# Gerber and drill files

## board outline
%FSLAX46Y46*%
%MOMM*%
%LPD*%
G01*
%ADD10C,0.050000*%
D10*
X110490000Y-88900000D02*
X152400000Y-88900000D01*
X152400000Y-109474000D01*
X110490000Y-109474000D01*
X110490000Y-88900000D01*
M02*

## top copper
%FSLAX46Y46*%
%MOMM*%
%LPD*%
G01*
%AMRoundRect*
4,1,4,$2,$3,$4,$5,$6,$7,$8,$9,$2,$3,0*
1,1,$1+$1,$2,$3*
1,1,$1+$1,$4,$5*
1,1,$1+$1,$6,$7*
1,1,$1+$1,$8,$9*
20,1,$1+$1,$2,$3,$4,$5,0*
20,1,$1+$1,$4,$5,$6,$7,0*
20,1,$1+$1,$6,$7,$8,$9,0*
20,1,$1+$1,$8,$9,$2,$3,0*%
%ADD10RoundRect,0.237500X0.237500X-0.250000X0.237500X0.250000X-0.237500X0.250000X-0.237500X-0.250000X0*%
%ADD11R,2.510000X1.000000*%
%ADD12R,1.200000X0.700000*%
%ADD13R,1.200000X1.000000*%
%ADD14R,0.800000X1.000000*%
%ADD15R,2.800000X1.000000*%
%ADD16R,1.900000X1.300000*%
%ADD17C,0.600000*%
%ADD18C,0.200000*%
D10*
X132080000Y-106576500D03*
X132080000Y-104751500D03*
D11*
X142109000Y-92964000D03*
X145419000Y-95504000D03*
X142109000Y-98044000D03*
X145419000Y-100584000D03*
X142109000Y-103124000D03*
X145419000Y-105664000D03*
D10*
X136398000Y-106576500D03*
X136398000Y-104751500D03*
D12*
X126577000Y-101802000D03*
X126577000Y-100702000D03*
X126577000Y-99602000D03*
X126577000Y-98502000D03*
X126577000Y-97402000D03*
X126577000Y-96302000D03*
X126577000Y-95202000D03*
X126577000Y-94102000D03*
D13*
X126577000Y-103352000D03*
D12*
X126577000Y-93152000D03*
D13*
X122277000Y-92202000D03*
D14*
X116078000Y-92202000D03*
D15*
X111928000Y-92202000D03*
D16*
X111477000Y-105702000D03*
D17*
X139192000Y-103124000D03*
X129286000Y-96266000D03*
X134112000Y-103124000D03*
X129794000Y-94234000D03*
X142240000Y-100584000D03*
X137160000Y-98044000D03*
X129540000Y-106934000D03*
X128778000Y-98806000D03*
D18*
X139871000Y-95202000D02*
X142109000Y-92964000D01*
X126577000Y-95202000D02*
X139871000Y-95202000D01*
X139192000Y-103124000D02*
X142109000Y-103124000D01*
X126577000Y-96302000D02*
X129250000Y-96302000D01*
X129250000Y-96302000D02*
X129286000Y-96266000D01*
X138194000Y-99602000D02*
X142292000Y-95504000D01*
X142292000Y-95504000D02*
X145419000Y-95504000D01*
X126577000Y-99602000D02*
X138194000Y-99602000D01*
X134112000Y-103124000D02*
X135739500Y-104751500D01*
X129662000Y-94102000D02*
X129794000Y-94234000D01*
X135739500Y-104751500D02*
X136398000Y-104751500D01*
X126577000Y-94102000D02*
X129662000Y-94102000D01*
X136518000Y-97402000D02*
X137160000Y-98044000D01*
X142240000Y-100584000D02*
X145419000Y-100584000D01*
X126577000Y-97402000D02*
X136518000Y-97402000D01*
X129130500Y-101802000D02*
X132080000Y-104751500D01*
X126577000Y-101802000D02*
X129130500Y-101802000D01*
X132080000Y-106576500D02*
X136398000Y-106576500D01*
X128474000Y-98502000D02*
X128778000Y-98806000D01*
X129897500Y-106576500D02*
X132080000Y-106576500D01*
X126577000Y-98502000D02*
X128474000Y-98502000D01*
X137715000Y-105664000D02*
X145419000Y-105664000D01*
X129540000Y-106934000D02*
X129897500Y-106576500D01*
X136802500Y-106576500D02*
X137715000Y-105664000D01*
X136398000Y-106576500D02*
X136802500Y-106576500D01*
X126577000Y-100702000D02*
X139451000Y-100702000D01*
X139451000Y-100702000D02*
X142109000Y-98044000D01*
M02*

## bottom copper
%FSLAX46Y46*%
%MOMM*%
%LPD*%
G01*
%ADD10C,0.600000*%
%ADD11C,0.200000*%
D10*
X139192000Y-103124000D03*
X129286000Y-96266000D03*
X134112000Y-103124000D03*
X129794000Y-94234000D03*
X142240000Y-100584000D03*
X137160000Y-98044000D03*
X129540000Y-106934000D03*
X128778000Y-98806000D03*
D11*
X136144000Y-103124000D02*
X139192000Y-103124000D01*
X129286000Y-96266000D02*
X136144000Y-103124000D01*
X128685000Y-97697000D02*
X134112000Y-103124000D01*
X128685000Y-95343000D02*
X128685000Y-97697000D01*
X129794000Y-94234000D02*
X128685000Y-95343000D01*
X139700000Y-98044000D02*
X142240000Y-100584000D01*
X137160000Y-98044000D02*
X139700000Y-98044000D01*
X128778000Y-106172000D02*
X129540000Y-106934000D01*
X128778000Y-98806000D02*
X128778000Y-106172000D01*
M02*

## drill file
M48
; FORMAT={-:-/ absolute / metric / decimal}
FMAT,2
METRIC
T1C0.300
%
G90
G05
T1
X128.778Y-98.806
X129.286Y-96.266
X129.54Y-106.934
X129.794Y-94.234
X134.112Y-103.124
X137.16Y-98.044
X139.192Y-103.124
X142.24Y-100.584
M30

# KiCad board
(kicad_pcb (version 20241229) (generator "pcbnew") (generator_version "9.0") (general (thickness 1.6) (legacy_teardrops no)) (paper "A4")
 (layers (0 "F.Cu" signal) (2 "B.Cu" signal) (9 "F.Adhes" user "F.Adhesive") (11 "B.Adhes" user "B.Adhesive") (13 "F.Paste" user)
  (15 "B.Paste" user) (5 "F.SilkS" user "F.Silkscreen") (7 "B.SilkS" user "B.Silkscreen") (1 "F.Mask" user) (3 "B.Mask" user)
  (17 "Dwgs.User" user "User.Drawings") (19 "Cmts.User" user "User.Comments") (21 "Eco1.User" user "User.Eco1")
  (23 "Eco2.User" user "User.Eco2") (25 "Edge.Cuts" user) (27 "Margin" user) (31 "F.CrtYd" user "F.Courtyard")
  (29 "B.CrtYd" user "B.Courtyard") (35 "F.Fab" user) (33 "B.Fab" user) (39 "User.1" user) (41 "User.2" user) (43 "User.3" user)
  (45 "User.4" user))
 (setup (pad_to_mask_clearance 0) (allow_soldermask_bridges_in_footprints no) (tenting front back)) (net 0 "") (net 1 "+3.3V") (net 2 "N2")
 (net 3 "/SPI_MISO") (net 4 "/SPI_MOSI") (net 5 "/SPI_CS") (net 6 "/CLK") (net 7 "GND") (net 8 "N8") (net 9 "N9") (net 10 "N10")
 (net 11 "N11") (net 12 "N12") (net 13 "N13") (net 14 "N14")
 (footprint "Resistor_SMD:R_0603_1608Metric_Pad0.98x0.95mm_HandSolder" (layer "F.Cu") (at 132.08 105.664 90)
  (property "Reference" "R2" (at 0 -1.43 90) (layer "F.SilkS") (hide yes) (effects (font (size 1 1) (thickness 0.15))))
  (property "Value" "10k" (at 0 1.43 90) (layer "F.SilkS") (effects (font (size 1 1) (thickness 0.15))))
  (pad "1" smd roundrect (at -0.9125 0 90) (size 0.975 0.95) (layers "F.Cu" "F.Mask" "F.Paste") (roundrect_rratio 0.25) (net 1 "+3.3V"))
  (pad "2" smd roundrect (at 0.9125 0 90) (size 0.975 0.95) (layers "F.Cu" "F.Mask" "F.Paste") (roundrect_rratio 0.25) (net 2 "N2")))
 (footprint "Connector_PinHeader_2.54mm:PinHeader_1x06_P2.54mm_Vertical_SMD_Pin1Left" (layer "F.Cu") (at 143.764 99.314)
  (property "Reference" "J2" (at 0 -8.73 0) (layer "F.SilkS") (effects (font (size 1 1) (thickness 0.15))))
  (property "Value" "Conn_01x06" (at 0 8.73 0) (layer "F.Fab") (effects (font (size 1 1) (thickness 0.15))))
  (pad "1" smd rect (at -1.655 -6.35) (size 2.51 1) (layers "F.Cu" "F.Mask" "F.Paste") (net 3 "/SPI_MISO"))
  (pad "2" smd rect (at 1.655 -3.81) (size 2.51 1) (layers "F.Cu" "F.Mask" "F.Paste") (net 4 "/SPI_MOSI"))
  (pad "3" smd rect (at -1.655 -1.27) (size 2.51 1) (layers "F.Cu" "F.Mask" "F.Paste") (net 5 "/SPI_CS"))
  (pad "4" smd rect (at 1.655 1.27) (size 2.51 1) (layers "F.Cu" "F.Mask" "F.Paste") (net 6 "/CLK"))
  (pad "5" smd rect (at -1.655 3.81) (size 2.51 1) (layers "F.Cu" "F.Mask" "F.Paste") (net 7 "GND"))
  (pad "6" smd rect (at 1.655 6.35) (size 2.51 1) (layers "F.Cu" "F.Mask" "F.Paste") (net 1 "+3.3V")))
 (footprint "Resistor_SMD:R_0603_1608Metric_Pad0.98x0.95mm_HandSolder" (layer "F.Cu") (at 136.398 105.664 90)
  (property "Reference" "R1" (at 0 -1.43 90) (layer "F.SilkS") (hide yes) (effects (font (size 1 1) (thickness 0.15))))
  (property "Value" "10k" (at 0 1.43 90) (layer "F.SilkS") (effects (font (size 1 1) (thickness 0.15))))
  (pad "1" smd roundrect (at -0.9125 0 90) (size 0.975 0.95) (layers "F.Cu" "F.Mask" "F.Paste") (roundrect_rratio 0.25) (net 1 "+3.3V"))
  (pad "2" smd roundrect (at 0.9125 0 90) (size 0.975 0.95) (layers "F.Cu" "F.Mask" "F.Paste") (roundrect_rratio 0.25) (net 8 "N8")))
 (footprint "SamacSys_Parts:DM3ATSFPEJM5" (layer "F.Cu") (at 119.165 99.027 -90)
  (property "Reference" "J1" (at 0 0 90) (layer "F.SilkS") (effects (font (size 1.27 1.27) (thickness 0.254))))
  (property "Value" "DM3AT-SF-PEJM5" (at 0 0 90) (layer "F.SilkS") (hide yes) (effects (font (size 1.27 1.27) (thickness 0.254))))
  (pad "1" smd rect (at 2.775 -7.412 270) (size 0.7 1.2) (layers "F.Cu" "F.Mask" "F.Paste") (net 2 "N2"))
  (pad "2" smd rect (at 1.675 -7.412 270) (size 0.7 1.2) (layers "F.Cu" "F.Mask" "F.Paste") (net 5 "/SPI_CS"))
  (pad "3" smd rect (at 0.575 -7.412 270) (size 0.7 1.2) (layers "F.Cu" "F.Mask" "F.Paste") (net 4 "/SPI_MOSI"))
  (pad "4" smd rect (at -0.525 -7.412 270) (size 0.7 1.2) (layers "F.Cu" "F.Mask" "F.Paste") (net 1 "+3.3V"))
  (pad "5" smd rect (at -1.625 -7.412 270) (size 0.7 1.2) (layers "F.Cu" "F.Mask" "F.Paste") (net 6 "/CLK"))
  (pad "6" smd rect (at -2.725 -7.412 270) (size 0.7 1.2) (layers "F.Cu" "F.Mask" "F.Paste") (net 7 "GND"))
  (pad "7" smd rect (at -3.825 -7.412 270) (size 0.7 1.2) (layers "F.Cu" "F.Mask" "F.Paste") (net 3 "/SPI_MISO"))
  (pad "8" smd rect (at -4.925 -7.412 270) (size 0.7 1.2) (layers "F.Cu" "F.Mask" "F.Paste") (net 8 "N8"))
  (pad "MP1" smd rect (at 4.325 -7.412 270) (size 1 1.2) (layers "F.Cu" "F.Mask" "F.Paste") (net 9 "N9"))
  (pad "MP2" smd rect (at -5.875 -7.412 270) (size 0.7 1.2) (layers "F.Cu" "F.Mask" "F.Paste") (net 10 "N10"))
  (pad "MP3" smd rect (at -6.825 -3.112 270) (size 1 1.2) (layers "F.Cu" "F.Mask" "F.Paste") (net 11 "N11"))
  (pad "MP4" smd rect (at -6.825 3.087) (size 0.8 1) (layers "F.Cu" "F.Mask" "F.Paste") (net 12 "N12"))
  (pad "MP5" smd rect (at -6.825 7.237 270) (size 1 2.8) (layers "F.Cu" "F.Mask" "F.Paste") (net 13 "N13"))
  (pad "MP6" smd rect (at 6.675 7.688 270) (size 1.3 1.9) (layers "F.Cu" "F.Mask" "F.Paste") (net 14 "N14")))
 (gr_rect (start 110.49 88.9) (end 152.4 109.474) (stroke (width 0.05) (type default)) (fill no) (layer "Edge.Cuts"))
 (segment (start 139.871 95.202) (end 142.109 92.964) (width 0.2) (layer "F.Cu") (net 3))
 (segment (start 126.577 95.202) (end 139.871 95.202) (width 0.2) (layer "F.Cu") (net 3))
 (segment (start 139.192 103.124) (end 142.109 103.124) (width 0.2) (layer "F.Cu") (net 7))
 (segment (start 126.577 96.302) (end 129.25 96.302) (width 0.2) (layer "F.Cu") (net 7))
 (segment (start 129.25 96.302) (end 129.286 96.266) (width 0.2) (layer "F.Cu") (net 7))
 (via (at 139.192 103.124) (size 0.6) (drill 0.3) (layers "F.Cu" "B.Cu") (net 7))
 (via (at 129.286 96.266) (size 0.6) (drill 0.3) (layers "F.Cu" "B.Cu") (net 7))
 (segment (start 136.144 103.124) (end 139.192 103.124) (width 0.2) (layer "B.Cu") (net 7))
 (segment (start 129.286 96.266) (end 136.144 103.124) (width 0.2) (layer "B.Cu") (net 7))
 (segment (start 138.194 99.602) (end 142.292 95.504) (width 0.2) (layer "F.Cu") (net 4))
 (segment (start 142.292 95.504) (end 145.419 95.504) (width 0.2) (layer "F.Cu") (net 4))
 (segment (start 126.577 99.602) (end 138.194 99.602) (width 0.2) (layer "F.Cu") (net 4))
 (segment (start 134.112 103.124) (end 135.7395 104.7515) (width 0.2) (layer "F.Cu") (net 8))
 (segment (start 129.662 94.102) (end 129.794 94.234) (width 0.2) (layer "F.Cu") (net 8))
 (segment (start 135.7395 104.7515) (end 136.398 104.7515) (width 0.2) (layer "F.Cu") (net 8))
 (segment (start 126.577 94.102) (end 129.662 94.102) (width 0.2) (layer "F.Cu") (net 8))
 (via (at 134.112 103.124) (size 0.6) (drill 0.3) (layers "F.Cu" "B.Cu") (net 8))
 (via (at 129.794 94.234) (size 0.6) (drill 0.3) (layers "F.Cu" "B.Cu") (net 8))
 (segment (start 128.685 97.697) (end 134.112 103.124) (width 0.2) (layer "B.Cu") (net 8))
 (segment (start 128.685 95.343) (end 128.685 97.697) (width 0.2) (layer "B.Cu") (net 8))
 (segment (start 129.794 94.234) (end 128.685 95.343) (width 0.2) (layer "B.Cu") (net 8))
 (segment (start 136.518 97.402) (end 137.16 98.044) (width 0.2) (layer "F.Cu") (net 6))
 (segment (start 142.24 100.584) (end 145.419 100.584) (width 0.2) (layer "F.Cu") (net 6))
 (segment (start 126.577 97.402) (end 136.518 97.402) (width 0.2) (layer "F.Cu") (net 6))
 (via (at 142.24 100.584) (size 0.6) (drill 0.3) (layers "F.Cu" "B.Cu") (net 6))
 (via (at 137.16 98.044) (size 0.6) (drill 0.3) (layers "F.Cu" "B.Cu") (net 6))
 (segment (start 139.7 98.044) (end 142.24 100.584) (width 0.2) (layer "B.Cu") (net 6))
 (segment (start 137.16 98.044) (end 139.7 98.044) (width 0.2) (layer "B.Cu") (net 6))
 (segment (start 129.1305 101.802) (end 132.08 104.7515) (width 0.2) (layer "F.Cu") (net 2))
 (segment (start 126.577 101.802) (end 129.1305 101.802) (width 0.2) (layer "F.Cu") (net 2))
 (segment (start 132.08 106.5765) (end 136.398 106.5765) (width 0.2) (layer "F.Cu") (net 1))
 (segment (start 128.474 98.502) (end 128.778 98.806) (width 0.2) (layer "F.Cu") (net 1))
 (segment (start 129.8975 106.5765) (end 132.08 106.5765) (width 0.2) (layer "F.Cu") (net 1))
 (segment (start 126.577 98.502) (end 128.474 98.502) (width 0.2) (layer "F.Cu") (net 1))
 (segment (start 137.715 105.664) (end 145.419 105.664) (width 0.2) (layer "F.Cu") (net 1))
 (segment (start 129.54 106.934) (end 129.8975 106.5765) (width 0.2) (layer "F.Cu") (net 1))
 (segment (start 136.8025 106.5765) (end 137.715 105.664) (width 0.2) (layer "F.Cu") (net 1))
 (segment (start 136.398 106.5765) (end 136.8025 106.5765) (width 0.2) (layer "F.Cu") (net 1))
 (via (at 129.54 106.934) (size 0.6) (drill 0.3) (layers "F.Cu" "B.Cu") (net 1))
 (via (at 128.778 98.806) (size 0.6) (drill 0.3) (layers "F.Cu" "B.Cu") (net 1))
 (segment (start 128.778 106.172) (end 129.54 106.934) (width 0.2) (layer "B.Cu") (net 1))
 (segment (start 128.778 98.806) (end 128.778 106.172) (width 0.2) (layer "B.Cu") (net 1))
 (segment (start 126.577 100.702) (end 139.451 100.702) (width 0.2) (layer "F.Cu") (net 5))
 (segment (start 139.451 100.702) (end 142.109 98.044) (width 0.2) (layer "F.Cu") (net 5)))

